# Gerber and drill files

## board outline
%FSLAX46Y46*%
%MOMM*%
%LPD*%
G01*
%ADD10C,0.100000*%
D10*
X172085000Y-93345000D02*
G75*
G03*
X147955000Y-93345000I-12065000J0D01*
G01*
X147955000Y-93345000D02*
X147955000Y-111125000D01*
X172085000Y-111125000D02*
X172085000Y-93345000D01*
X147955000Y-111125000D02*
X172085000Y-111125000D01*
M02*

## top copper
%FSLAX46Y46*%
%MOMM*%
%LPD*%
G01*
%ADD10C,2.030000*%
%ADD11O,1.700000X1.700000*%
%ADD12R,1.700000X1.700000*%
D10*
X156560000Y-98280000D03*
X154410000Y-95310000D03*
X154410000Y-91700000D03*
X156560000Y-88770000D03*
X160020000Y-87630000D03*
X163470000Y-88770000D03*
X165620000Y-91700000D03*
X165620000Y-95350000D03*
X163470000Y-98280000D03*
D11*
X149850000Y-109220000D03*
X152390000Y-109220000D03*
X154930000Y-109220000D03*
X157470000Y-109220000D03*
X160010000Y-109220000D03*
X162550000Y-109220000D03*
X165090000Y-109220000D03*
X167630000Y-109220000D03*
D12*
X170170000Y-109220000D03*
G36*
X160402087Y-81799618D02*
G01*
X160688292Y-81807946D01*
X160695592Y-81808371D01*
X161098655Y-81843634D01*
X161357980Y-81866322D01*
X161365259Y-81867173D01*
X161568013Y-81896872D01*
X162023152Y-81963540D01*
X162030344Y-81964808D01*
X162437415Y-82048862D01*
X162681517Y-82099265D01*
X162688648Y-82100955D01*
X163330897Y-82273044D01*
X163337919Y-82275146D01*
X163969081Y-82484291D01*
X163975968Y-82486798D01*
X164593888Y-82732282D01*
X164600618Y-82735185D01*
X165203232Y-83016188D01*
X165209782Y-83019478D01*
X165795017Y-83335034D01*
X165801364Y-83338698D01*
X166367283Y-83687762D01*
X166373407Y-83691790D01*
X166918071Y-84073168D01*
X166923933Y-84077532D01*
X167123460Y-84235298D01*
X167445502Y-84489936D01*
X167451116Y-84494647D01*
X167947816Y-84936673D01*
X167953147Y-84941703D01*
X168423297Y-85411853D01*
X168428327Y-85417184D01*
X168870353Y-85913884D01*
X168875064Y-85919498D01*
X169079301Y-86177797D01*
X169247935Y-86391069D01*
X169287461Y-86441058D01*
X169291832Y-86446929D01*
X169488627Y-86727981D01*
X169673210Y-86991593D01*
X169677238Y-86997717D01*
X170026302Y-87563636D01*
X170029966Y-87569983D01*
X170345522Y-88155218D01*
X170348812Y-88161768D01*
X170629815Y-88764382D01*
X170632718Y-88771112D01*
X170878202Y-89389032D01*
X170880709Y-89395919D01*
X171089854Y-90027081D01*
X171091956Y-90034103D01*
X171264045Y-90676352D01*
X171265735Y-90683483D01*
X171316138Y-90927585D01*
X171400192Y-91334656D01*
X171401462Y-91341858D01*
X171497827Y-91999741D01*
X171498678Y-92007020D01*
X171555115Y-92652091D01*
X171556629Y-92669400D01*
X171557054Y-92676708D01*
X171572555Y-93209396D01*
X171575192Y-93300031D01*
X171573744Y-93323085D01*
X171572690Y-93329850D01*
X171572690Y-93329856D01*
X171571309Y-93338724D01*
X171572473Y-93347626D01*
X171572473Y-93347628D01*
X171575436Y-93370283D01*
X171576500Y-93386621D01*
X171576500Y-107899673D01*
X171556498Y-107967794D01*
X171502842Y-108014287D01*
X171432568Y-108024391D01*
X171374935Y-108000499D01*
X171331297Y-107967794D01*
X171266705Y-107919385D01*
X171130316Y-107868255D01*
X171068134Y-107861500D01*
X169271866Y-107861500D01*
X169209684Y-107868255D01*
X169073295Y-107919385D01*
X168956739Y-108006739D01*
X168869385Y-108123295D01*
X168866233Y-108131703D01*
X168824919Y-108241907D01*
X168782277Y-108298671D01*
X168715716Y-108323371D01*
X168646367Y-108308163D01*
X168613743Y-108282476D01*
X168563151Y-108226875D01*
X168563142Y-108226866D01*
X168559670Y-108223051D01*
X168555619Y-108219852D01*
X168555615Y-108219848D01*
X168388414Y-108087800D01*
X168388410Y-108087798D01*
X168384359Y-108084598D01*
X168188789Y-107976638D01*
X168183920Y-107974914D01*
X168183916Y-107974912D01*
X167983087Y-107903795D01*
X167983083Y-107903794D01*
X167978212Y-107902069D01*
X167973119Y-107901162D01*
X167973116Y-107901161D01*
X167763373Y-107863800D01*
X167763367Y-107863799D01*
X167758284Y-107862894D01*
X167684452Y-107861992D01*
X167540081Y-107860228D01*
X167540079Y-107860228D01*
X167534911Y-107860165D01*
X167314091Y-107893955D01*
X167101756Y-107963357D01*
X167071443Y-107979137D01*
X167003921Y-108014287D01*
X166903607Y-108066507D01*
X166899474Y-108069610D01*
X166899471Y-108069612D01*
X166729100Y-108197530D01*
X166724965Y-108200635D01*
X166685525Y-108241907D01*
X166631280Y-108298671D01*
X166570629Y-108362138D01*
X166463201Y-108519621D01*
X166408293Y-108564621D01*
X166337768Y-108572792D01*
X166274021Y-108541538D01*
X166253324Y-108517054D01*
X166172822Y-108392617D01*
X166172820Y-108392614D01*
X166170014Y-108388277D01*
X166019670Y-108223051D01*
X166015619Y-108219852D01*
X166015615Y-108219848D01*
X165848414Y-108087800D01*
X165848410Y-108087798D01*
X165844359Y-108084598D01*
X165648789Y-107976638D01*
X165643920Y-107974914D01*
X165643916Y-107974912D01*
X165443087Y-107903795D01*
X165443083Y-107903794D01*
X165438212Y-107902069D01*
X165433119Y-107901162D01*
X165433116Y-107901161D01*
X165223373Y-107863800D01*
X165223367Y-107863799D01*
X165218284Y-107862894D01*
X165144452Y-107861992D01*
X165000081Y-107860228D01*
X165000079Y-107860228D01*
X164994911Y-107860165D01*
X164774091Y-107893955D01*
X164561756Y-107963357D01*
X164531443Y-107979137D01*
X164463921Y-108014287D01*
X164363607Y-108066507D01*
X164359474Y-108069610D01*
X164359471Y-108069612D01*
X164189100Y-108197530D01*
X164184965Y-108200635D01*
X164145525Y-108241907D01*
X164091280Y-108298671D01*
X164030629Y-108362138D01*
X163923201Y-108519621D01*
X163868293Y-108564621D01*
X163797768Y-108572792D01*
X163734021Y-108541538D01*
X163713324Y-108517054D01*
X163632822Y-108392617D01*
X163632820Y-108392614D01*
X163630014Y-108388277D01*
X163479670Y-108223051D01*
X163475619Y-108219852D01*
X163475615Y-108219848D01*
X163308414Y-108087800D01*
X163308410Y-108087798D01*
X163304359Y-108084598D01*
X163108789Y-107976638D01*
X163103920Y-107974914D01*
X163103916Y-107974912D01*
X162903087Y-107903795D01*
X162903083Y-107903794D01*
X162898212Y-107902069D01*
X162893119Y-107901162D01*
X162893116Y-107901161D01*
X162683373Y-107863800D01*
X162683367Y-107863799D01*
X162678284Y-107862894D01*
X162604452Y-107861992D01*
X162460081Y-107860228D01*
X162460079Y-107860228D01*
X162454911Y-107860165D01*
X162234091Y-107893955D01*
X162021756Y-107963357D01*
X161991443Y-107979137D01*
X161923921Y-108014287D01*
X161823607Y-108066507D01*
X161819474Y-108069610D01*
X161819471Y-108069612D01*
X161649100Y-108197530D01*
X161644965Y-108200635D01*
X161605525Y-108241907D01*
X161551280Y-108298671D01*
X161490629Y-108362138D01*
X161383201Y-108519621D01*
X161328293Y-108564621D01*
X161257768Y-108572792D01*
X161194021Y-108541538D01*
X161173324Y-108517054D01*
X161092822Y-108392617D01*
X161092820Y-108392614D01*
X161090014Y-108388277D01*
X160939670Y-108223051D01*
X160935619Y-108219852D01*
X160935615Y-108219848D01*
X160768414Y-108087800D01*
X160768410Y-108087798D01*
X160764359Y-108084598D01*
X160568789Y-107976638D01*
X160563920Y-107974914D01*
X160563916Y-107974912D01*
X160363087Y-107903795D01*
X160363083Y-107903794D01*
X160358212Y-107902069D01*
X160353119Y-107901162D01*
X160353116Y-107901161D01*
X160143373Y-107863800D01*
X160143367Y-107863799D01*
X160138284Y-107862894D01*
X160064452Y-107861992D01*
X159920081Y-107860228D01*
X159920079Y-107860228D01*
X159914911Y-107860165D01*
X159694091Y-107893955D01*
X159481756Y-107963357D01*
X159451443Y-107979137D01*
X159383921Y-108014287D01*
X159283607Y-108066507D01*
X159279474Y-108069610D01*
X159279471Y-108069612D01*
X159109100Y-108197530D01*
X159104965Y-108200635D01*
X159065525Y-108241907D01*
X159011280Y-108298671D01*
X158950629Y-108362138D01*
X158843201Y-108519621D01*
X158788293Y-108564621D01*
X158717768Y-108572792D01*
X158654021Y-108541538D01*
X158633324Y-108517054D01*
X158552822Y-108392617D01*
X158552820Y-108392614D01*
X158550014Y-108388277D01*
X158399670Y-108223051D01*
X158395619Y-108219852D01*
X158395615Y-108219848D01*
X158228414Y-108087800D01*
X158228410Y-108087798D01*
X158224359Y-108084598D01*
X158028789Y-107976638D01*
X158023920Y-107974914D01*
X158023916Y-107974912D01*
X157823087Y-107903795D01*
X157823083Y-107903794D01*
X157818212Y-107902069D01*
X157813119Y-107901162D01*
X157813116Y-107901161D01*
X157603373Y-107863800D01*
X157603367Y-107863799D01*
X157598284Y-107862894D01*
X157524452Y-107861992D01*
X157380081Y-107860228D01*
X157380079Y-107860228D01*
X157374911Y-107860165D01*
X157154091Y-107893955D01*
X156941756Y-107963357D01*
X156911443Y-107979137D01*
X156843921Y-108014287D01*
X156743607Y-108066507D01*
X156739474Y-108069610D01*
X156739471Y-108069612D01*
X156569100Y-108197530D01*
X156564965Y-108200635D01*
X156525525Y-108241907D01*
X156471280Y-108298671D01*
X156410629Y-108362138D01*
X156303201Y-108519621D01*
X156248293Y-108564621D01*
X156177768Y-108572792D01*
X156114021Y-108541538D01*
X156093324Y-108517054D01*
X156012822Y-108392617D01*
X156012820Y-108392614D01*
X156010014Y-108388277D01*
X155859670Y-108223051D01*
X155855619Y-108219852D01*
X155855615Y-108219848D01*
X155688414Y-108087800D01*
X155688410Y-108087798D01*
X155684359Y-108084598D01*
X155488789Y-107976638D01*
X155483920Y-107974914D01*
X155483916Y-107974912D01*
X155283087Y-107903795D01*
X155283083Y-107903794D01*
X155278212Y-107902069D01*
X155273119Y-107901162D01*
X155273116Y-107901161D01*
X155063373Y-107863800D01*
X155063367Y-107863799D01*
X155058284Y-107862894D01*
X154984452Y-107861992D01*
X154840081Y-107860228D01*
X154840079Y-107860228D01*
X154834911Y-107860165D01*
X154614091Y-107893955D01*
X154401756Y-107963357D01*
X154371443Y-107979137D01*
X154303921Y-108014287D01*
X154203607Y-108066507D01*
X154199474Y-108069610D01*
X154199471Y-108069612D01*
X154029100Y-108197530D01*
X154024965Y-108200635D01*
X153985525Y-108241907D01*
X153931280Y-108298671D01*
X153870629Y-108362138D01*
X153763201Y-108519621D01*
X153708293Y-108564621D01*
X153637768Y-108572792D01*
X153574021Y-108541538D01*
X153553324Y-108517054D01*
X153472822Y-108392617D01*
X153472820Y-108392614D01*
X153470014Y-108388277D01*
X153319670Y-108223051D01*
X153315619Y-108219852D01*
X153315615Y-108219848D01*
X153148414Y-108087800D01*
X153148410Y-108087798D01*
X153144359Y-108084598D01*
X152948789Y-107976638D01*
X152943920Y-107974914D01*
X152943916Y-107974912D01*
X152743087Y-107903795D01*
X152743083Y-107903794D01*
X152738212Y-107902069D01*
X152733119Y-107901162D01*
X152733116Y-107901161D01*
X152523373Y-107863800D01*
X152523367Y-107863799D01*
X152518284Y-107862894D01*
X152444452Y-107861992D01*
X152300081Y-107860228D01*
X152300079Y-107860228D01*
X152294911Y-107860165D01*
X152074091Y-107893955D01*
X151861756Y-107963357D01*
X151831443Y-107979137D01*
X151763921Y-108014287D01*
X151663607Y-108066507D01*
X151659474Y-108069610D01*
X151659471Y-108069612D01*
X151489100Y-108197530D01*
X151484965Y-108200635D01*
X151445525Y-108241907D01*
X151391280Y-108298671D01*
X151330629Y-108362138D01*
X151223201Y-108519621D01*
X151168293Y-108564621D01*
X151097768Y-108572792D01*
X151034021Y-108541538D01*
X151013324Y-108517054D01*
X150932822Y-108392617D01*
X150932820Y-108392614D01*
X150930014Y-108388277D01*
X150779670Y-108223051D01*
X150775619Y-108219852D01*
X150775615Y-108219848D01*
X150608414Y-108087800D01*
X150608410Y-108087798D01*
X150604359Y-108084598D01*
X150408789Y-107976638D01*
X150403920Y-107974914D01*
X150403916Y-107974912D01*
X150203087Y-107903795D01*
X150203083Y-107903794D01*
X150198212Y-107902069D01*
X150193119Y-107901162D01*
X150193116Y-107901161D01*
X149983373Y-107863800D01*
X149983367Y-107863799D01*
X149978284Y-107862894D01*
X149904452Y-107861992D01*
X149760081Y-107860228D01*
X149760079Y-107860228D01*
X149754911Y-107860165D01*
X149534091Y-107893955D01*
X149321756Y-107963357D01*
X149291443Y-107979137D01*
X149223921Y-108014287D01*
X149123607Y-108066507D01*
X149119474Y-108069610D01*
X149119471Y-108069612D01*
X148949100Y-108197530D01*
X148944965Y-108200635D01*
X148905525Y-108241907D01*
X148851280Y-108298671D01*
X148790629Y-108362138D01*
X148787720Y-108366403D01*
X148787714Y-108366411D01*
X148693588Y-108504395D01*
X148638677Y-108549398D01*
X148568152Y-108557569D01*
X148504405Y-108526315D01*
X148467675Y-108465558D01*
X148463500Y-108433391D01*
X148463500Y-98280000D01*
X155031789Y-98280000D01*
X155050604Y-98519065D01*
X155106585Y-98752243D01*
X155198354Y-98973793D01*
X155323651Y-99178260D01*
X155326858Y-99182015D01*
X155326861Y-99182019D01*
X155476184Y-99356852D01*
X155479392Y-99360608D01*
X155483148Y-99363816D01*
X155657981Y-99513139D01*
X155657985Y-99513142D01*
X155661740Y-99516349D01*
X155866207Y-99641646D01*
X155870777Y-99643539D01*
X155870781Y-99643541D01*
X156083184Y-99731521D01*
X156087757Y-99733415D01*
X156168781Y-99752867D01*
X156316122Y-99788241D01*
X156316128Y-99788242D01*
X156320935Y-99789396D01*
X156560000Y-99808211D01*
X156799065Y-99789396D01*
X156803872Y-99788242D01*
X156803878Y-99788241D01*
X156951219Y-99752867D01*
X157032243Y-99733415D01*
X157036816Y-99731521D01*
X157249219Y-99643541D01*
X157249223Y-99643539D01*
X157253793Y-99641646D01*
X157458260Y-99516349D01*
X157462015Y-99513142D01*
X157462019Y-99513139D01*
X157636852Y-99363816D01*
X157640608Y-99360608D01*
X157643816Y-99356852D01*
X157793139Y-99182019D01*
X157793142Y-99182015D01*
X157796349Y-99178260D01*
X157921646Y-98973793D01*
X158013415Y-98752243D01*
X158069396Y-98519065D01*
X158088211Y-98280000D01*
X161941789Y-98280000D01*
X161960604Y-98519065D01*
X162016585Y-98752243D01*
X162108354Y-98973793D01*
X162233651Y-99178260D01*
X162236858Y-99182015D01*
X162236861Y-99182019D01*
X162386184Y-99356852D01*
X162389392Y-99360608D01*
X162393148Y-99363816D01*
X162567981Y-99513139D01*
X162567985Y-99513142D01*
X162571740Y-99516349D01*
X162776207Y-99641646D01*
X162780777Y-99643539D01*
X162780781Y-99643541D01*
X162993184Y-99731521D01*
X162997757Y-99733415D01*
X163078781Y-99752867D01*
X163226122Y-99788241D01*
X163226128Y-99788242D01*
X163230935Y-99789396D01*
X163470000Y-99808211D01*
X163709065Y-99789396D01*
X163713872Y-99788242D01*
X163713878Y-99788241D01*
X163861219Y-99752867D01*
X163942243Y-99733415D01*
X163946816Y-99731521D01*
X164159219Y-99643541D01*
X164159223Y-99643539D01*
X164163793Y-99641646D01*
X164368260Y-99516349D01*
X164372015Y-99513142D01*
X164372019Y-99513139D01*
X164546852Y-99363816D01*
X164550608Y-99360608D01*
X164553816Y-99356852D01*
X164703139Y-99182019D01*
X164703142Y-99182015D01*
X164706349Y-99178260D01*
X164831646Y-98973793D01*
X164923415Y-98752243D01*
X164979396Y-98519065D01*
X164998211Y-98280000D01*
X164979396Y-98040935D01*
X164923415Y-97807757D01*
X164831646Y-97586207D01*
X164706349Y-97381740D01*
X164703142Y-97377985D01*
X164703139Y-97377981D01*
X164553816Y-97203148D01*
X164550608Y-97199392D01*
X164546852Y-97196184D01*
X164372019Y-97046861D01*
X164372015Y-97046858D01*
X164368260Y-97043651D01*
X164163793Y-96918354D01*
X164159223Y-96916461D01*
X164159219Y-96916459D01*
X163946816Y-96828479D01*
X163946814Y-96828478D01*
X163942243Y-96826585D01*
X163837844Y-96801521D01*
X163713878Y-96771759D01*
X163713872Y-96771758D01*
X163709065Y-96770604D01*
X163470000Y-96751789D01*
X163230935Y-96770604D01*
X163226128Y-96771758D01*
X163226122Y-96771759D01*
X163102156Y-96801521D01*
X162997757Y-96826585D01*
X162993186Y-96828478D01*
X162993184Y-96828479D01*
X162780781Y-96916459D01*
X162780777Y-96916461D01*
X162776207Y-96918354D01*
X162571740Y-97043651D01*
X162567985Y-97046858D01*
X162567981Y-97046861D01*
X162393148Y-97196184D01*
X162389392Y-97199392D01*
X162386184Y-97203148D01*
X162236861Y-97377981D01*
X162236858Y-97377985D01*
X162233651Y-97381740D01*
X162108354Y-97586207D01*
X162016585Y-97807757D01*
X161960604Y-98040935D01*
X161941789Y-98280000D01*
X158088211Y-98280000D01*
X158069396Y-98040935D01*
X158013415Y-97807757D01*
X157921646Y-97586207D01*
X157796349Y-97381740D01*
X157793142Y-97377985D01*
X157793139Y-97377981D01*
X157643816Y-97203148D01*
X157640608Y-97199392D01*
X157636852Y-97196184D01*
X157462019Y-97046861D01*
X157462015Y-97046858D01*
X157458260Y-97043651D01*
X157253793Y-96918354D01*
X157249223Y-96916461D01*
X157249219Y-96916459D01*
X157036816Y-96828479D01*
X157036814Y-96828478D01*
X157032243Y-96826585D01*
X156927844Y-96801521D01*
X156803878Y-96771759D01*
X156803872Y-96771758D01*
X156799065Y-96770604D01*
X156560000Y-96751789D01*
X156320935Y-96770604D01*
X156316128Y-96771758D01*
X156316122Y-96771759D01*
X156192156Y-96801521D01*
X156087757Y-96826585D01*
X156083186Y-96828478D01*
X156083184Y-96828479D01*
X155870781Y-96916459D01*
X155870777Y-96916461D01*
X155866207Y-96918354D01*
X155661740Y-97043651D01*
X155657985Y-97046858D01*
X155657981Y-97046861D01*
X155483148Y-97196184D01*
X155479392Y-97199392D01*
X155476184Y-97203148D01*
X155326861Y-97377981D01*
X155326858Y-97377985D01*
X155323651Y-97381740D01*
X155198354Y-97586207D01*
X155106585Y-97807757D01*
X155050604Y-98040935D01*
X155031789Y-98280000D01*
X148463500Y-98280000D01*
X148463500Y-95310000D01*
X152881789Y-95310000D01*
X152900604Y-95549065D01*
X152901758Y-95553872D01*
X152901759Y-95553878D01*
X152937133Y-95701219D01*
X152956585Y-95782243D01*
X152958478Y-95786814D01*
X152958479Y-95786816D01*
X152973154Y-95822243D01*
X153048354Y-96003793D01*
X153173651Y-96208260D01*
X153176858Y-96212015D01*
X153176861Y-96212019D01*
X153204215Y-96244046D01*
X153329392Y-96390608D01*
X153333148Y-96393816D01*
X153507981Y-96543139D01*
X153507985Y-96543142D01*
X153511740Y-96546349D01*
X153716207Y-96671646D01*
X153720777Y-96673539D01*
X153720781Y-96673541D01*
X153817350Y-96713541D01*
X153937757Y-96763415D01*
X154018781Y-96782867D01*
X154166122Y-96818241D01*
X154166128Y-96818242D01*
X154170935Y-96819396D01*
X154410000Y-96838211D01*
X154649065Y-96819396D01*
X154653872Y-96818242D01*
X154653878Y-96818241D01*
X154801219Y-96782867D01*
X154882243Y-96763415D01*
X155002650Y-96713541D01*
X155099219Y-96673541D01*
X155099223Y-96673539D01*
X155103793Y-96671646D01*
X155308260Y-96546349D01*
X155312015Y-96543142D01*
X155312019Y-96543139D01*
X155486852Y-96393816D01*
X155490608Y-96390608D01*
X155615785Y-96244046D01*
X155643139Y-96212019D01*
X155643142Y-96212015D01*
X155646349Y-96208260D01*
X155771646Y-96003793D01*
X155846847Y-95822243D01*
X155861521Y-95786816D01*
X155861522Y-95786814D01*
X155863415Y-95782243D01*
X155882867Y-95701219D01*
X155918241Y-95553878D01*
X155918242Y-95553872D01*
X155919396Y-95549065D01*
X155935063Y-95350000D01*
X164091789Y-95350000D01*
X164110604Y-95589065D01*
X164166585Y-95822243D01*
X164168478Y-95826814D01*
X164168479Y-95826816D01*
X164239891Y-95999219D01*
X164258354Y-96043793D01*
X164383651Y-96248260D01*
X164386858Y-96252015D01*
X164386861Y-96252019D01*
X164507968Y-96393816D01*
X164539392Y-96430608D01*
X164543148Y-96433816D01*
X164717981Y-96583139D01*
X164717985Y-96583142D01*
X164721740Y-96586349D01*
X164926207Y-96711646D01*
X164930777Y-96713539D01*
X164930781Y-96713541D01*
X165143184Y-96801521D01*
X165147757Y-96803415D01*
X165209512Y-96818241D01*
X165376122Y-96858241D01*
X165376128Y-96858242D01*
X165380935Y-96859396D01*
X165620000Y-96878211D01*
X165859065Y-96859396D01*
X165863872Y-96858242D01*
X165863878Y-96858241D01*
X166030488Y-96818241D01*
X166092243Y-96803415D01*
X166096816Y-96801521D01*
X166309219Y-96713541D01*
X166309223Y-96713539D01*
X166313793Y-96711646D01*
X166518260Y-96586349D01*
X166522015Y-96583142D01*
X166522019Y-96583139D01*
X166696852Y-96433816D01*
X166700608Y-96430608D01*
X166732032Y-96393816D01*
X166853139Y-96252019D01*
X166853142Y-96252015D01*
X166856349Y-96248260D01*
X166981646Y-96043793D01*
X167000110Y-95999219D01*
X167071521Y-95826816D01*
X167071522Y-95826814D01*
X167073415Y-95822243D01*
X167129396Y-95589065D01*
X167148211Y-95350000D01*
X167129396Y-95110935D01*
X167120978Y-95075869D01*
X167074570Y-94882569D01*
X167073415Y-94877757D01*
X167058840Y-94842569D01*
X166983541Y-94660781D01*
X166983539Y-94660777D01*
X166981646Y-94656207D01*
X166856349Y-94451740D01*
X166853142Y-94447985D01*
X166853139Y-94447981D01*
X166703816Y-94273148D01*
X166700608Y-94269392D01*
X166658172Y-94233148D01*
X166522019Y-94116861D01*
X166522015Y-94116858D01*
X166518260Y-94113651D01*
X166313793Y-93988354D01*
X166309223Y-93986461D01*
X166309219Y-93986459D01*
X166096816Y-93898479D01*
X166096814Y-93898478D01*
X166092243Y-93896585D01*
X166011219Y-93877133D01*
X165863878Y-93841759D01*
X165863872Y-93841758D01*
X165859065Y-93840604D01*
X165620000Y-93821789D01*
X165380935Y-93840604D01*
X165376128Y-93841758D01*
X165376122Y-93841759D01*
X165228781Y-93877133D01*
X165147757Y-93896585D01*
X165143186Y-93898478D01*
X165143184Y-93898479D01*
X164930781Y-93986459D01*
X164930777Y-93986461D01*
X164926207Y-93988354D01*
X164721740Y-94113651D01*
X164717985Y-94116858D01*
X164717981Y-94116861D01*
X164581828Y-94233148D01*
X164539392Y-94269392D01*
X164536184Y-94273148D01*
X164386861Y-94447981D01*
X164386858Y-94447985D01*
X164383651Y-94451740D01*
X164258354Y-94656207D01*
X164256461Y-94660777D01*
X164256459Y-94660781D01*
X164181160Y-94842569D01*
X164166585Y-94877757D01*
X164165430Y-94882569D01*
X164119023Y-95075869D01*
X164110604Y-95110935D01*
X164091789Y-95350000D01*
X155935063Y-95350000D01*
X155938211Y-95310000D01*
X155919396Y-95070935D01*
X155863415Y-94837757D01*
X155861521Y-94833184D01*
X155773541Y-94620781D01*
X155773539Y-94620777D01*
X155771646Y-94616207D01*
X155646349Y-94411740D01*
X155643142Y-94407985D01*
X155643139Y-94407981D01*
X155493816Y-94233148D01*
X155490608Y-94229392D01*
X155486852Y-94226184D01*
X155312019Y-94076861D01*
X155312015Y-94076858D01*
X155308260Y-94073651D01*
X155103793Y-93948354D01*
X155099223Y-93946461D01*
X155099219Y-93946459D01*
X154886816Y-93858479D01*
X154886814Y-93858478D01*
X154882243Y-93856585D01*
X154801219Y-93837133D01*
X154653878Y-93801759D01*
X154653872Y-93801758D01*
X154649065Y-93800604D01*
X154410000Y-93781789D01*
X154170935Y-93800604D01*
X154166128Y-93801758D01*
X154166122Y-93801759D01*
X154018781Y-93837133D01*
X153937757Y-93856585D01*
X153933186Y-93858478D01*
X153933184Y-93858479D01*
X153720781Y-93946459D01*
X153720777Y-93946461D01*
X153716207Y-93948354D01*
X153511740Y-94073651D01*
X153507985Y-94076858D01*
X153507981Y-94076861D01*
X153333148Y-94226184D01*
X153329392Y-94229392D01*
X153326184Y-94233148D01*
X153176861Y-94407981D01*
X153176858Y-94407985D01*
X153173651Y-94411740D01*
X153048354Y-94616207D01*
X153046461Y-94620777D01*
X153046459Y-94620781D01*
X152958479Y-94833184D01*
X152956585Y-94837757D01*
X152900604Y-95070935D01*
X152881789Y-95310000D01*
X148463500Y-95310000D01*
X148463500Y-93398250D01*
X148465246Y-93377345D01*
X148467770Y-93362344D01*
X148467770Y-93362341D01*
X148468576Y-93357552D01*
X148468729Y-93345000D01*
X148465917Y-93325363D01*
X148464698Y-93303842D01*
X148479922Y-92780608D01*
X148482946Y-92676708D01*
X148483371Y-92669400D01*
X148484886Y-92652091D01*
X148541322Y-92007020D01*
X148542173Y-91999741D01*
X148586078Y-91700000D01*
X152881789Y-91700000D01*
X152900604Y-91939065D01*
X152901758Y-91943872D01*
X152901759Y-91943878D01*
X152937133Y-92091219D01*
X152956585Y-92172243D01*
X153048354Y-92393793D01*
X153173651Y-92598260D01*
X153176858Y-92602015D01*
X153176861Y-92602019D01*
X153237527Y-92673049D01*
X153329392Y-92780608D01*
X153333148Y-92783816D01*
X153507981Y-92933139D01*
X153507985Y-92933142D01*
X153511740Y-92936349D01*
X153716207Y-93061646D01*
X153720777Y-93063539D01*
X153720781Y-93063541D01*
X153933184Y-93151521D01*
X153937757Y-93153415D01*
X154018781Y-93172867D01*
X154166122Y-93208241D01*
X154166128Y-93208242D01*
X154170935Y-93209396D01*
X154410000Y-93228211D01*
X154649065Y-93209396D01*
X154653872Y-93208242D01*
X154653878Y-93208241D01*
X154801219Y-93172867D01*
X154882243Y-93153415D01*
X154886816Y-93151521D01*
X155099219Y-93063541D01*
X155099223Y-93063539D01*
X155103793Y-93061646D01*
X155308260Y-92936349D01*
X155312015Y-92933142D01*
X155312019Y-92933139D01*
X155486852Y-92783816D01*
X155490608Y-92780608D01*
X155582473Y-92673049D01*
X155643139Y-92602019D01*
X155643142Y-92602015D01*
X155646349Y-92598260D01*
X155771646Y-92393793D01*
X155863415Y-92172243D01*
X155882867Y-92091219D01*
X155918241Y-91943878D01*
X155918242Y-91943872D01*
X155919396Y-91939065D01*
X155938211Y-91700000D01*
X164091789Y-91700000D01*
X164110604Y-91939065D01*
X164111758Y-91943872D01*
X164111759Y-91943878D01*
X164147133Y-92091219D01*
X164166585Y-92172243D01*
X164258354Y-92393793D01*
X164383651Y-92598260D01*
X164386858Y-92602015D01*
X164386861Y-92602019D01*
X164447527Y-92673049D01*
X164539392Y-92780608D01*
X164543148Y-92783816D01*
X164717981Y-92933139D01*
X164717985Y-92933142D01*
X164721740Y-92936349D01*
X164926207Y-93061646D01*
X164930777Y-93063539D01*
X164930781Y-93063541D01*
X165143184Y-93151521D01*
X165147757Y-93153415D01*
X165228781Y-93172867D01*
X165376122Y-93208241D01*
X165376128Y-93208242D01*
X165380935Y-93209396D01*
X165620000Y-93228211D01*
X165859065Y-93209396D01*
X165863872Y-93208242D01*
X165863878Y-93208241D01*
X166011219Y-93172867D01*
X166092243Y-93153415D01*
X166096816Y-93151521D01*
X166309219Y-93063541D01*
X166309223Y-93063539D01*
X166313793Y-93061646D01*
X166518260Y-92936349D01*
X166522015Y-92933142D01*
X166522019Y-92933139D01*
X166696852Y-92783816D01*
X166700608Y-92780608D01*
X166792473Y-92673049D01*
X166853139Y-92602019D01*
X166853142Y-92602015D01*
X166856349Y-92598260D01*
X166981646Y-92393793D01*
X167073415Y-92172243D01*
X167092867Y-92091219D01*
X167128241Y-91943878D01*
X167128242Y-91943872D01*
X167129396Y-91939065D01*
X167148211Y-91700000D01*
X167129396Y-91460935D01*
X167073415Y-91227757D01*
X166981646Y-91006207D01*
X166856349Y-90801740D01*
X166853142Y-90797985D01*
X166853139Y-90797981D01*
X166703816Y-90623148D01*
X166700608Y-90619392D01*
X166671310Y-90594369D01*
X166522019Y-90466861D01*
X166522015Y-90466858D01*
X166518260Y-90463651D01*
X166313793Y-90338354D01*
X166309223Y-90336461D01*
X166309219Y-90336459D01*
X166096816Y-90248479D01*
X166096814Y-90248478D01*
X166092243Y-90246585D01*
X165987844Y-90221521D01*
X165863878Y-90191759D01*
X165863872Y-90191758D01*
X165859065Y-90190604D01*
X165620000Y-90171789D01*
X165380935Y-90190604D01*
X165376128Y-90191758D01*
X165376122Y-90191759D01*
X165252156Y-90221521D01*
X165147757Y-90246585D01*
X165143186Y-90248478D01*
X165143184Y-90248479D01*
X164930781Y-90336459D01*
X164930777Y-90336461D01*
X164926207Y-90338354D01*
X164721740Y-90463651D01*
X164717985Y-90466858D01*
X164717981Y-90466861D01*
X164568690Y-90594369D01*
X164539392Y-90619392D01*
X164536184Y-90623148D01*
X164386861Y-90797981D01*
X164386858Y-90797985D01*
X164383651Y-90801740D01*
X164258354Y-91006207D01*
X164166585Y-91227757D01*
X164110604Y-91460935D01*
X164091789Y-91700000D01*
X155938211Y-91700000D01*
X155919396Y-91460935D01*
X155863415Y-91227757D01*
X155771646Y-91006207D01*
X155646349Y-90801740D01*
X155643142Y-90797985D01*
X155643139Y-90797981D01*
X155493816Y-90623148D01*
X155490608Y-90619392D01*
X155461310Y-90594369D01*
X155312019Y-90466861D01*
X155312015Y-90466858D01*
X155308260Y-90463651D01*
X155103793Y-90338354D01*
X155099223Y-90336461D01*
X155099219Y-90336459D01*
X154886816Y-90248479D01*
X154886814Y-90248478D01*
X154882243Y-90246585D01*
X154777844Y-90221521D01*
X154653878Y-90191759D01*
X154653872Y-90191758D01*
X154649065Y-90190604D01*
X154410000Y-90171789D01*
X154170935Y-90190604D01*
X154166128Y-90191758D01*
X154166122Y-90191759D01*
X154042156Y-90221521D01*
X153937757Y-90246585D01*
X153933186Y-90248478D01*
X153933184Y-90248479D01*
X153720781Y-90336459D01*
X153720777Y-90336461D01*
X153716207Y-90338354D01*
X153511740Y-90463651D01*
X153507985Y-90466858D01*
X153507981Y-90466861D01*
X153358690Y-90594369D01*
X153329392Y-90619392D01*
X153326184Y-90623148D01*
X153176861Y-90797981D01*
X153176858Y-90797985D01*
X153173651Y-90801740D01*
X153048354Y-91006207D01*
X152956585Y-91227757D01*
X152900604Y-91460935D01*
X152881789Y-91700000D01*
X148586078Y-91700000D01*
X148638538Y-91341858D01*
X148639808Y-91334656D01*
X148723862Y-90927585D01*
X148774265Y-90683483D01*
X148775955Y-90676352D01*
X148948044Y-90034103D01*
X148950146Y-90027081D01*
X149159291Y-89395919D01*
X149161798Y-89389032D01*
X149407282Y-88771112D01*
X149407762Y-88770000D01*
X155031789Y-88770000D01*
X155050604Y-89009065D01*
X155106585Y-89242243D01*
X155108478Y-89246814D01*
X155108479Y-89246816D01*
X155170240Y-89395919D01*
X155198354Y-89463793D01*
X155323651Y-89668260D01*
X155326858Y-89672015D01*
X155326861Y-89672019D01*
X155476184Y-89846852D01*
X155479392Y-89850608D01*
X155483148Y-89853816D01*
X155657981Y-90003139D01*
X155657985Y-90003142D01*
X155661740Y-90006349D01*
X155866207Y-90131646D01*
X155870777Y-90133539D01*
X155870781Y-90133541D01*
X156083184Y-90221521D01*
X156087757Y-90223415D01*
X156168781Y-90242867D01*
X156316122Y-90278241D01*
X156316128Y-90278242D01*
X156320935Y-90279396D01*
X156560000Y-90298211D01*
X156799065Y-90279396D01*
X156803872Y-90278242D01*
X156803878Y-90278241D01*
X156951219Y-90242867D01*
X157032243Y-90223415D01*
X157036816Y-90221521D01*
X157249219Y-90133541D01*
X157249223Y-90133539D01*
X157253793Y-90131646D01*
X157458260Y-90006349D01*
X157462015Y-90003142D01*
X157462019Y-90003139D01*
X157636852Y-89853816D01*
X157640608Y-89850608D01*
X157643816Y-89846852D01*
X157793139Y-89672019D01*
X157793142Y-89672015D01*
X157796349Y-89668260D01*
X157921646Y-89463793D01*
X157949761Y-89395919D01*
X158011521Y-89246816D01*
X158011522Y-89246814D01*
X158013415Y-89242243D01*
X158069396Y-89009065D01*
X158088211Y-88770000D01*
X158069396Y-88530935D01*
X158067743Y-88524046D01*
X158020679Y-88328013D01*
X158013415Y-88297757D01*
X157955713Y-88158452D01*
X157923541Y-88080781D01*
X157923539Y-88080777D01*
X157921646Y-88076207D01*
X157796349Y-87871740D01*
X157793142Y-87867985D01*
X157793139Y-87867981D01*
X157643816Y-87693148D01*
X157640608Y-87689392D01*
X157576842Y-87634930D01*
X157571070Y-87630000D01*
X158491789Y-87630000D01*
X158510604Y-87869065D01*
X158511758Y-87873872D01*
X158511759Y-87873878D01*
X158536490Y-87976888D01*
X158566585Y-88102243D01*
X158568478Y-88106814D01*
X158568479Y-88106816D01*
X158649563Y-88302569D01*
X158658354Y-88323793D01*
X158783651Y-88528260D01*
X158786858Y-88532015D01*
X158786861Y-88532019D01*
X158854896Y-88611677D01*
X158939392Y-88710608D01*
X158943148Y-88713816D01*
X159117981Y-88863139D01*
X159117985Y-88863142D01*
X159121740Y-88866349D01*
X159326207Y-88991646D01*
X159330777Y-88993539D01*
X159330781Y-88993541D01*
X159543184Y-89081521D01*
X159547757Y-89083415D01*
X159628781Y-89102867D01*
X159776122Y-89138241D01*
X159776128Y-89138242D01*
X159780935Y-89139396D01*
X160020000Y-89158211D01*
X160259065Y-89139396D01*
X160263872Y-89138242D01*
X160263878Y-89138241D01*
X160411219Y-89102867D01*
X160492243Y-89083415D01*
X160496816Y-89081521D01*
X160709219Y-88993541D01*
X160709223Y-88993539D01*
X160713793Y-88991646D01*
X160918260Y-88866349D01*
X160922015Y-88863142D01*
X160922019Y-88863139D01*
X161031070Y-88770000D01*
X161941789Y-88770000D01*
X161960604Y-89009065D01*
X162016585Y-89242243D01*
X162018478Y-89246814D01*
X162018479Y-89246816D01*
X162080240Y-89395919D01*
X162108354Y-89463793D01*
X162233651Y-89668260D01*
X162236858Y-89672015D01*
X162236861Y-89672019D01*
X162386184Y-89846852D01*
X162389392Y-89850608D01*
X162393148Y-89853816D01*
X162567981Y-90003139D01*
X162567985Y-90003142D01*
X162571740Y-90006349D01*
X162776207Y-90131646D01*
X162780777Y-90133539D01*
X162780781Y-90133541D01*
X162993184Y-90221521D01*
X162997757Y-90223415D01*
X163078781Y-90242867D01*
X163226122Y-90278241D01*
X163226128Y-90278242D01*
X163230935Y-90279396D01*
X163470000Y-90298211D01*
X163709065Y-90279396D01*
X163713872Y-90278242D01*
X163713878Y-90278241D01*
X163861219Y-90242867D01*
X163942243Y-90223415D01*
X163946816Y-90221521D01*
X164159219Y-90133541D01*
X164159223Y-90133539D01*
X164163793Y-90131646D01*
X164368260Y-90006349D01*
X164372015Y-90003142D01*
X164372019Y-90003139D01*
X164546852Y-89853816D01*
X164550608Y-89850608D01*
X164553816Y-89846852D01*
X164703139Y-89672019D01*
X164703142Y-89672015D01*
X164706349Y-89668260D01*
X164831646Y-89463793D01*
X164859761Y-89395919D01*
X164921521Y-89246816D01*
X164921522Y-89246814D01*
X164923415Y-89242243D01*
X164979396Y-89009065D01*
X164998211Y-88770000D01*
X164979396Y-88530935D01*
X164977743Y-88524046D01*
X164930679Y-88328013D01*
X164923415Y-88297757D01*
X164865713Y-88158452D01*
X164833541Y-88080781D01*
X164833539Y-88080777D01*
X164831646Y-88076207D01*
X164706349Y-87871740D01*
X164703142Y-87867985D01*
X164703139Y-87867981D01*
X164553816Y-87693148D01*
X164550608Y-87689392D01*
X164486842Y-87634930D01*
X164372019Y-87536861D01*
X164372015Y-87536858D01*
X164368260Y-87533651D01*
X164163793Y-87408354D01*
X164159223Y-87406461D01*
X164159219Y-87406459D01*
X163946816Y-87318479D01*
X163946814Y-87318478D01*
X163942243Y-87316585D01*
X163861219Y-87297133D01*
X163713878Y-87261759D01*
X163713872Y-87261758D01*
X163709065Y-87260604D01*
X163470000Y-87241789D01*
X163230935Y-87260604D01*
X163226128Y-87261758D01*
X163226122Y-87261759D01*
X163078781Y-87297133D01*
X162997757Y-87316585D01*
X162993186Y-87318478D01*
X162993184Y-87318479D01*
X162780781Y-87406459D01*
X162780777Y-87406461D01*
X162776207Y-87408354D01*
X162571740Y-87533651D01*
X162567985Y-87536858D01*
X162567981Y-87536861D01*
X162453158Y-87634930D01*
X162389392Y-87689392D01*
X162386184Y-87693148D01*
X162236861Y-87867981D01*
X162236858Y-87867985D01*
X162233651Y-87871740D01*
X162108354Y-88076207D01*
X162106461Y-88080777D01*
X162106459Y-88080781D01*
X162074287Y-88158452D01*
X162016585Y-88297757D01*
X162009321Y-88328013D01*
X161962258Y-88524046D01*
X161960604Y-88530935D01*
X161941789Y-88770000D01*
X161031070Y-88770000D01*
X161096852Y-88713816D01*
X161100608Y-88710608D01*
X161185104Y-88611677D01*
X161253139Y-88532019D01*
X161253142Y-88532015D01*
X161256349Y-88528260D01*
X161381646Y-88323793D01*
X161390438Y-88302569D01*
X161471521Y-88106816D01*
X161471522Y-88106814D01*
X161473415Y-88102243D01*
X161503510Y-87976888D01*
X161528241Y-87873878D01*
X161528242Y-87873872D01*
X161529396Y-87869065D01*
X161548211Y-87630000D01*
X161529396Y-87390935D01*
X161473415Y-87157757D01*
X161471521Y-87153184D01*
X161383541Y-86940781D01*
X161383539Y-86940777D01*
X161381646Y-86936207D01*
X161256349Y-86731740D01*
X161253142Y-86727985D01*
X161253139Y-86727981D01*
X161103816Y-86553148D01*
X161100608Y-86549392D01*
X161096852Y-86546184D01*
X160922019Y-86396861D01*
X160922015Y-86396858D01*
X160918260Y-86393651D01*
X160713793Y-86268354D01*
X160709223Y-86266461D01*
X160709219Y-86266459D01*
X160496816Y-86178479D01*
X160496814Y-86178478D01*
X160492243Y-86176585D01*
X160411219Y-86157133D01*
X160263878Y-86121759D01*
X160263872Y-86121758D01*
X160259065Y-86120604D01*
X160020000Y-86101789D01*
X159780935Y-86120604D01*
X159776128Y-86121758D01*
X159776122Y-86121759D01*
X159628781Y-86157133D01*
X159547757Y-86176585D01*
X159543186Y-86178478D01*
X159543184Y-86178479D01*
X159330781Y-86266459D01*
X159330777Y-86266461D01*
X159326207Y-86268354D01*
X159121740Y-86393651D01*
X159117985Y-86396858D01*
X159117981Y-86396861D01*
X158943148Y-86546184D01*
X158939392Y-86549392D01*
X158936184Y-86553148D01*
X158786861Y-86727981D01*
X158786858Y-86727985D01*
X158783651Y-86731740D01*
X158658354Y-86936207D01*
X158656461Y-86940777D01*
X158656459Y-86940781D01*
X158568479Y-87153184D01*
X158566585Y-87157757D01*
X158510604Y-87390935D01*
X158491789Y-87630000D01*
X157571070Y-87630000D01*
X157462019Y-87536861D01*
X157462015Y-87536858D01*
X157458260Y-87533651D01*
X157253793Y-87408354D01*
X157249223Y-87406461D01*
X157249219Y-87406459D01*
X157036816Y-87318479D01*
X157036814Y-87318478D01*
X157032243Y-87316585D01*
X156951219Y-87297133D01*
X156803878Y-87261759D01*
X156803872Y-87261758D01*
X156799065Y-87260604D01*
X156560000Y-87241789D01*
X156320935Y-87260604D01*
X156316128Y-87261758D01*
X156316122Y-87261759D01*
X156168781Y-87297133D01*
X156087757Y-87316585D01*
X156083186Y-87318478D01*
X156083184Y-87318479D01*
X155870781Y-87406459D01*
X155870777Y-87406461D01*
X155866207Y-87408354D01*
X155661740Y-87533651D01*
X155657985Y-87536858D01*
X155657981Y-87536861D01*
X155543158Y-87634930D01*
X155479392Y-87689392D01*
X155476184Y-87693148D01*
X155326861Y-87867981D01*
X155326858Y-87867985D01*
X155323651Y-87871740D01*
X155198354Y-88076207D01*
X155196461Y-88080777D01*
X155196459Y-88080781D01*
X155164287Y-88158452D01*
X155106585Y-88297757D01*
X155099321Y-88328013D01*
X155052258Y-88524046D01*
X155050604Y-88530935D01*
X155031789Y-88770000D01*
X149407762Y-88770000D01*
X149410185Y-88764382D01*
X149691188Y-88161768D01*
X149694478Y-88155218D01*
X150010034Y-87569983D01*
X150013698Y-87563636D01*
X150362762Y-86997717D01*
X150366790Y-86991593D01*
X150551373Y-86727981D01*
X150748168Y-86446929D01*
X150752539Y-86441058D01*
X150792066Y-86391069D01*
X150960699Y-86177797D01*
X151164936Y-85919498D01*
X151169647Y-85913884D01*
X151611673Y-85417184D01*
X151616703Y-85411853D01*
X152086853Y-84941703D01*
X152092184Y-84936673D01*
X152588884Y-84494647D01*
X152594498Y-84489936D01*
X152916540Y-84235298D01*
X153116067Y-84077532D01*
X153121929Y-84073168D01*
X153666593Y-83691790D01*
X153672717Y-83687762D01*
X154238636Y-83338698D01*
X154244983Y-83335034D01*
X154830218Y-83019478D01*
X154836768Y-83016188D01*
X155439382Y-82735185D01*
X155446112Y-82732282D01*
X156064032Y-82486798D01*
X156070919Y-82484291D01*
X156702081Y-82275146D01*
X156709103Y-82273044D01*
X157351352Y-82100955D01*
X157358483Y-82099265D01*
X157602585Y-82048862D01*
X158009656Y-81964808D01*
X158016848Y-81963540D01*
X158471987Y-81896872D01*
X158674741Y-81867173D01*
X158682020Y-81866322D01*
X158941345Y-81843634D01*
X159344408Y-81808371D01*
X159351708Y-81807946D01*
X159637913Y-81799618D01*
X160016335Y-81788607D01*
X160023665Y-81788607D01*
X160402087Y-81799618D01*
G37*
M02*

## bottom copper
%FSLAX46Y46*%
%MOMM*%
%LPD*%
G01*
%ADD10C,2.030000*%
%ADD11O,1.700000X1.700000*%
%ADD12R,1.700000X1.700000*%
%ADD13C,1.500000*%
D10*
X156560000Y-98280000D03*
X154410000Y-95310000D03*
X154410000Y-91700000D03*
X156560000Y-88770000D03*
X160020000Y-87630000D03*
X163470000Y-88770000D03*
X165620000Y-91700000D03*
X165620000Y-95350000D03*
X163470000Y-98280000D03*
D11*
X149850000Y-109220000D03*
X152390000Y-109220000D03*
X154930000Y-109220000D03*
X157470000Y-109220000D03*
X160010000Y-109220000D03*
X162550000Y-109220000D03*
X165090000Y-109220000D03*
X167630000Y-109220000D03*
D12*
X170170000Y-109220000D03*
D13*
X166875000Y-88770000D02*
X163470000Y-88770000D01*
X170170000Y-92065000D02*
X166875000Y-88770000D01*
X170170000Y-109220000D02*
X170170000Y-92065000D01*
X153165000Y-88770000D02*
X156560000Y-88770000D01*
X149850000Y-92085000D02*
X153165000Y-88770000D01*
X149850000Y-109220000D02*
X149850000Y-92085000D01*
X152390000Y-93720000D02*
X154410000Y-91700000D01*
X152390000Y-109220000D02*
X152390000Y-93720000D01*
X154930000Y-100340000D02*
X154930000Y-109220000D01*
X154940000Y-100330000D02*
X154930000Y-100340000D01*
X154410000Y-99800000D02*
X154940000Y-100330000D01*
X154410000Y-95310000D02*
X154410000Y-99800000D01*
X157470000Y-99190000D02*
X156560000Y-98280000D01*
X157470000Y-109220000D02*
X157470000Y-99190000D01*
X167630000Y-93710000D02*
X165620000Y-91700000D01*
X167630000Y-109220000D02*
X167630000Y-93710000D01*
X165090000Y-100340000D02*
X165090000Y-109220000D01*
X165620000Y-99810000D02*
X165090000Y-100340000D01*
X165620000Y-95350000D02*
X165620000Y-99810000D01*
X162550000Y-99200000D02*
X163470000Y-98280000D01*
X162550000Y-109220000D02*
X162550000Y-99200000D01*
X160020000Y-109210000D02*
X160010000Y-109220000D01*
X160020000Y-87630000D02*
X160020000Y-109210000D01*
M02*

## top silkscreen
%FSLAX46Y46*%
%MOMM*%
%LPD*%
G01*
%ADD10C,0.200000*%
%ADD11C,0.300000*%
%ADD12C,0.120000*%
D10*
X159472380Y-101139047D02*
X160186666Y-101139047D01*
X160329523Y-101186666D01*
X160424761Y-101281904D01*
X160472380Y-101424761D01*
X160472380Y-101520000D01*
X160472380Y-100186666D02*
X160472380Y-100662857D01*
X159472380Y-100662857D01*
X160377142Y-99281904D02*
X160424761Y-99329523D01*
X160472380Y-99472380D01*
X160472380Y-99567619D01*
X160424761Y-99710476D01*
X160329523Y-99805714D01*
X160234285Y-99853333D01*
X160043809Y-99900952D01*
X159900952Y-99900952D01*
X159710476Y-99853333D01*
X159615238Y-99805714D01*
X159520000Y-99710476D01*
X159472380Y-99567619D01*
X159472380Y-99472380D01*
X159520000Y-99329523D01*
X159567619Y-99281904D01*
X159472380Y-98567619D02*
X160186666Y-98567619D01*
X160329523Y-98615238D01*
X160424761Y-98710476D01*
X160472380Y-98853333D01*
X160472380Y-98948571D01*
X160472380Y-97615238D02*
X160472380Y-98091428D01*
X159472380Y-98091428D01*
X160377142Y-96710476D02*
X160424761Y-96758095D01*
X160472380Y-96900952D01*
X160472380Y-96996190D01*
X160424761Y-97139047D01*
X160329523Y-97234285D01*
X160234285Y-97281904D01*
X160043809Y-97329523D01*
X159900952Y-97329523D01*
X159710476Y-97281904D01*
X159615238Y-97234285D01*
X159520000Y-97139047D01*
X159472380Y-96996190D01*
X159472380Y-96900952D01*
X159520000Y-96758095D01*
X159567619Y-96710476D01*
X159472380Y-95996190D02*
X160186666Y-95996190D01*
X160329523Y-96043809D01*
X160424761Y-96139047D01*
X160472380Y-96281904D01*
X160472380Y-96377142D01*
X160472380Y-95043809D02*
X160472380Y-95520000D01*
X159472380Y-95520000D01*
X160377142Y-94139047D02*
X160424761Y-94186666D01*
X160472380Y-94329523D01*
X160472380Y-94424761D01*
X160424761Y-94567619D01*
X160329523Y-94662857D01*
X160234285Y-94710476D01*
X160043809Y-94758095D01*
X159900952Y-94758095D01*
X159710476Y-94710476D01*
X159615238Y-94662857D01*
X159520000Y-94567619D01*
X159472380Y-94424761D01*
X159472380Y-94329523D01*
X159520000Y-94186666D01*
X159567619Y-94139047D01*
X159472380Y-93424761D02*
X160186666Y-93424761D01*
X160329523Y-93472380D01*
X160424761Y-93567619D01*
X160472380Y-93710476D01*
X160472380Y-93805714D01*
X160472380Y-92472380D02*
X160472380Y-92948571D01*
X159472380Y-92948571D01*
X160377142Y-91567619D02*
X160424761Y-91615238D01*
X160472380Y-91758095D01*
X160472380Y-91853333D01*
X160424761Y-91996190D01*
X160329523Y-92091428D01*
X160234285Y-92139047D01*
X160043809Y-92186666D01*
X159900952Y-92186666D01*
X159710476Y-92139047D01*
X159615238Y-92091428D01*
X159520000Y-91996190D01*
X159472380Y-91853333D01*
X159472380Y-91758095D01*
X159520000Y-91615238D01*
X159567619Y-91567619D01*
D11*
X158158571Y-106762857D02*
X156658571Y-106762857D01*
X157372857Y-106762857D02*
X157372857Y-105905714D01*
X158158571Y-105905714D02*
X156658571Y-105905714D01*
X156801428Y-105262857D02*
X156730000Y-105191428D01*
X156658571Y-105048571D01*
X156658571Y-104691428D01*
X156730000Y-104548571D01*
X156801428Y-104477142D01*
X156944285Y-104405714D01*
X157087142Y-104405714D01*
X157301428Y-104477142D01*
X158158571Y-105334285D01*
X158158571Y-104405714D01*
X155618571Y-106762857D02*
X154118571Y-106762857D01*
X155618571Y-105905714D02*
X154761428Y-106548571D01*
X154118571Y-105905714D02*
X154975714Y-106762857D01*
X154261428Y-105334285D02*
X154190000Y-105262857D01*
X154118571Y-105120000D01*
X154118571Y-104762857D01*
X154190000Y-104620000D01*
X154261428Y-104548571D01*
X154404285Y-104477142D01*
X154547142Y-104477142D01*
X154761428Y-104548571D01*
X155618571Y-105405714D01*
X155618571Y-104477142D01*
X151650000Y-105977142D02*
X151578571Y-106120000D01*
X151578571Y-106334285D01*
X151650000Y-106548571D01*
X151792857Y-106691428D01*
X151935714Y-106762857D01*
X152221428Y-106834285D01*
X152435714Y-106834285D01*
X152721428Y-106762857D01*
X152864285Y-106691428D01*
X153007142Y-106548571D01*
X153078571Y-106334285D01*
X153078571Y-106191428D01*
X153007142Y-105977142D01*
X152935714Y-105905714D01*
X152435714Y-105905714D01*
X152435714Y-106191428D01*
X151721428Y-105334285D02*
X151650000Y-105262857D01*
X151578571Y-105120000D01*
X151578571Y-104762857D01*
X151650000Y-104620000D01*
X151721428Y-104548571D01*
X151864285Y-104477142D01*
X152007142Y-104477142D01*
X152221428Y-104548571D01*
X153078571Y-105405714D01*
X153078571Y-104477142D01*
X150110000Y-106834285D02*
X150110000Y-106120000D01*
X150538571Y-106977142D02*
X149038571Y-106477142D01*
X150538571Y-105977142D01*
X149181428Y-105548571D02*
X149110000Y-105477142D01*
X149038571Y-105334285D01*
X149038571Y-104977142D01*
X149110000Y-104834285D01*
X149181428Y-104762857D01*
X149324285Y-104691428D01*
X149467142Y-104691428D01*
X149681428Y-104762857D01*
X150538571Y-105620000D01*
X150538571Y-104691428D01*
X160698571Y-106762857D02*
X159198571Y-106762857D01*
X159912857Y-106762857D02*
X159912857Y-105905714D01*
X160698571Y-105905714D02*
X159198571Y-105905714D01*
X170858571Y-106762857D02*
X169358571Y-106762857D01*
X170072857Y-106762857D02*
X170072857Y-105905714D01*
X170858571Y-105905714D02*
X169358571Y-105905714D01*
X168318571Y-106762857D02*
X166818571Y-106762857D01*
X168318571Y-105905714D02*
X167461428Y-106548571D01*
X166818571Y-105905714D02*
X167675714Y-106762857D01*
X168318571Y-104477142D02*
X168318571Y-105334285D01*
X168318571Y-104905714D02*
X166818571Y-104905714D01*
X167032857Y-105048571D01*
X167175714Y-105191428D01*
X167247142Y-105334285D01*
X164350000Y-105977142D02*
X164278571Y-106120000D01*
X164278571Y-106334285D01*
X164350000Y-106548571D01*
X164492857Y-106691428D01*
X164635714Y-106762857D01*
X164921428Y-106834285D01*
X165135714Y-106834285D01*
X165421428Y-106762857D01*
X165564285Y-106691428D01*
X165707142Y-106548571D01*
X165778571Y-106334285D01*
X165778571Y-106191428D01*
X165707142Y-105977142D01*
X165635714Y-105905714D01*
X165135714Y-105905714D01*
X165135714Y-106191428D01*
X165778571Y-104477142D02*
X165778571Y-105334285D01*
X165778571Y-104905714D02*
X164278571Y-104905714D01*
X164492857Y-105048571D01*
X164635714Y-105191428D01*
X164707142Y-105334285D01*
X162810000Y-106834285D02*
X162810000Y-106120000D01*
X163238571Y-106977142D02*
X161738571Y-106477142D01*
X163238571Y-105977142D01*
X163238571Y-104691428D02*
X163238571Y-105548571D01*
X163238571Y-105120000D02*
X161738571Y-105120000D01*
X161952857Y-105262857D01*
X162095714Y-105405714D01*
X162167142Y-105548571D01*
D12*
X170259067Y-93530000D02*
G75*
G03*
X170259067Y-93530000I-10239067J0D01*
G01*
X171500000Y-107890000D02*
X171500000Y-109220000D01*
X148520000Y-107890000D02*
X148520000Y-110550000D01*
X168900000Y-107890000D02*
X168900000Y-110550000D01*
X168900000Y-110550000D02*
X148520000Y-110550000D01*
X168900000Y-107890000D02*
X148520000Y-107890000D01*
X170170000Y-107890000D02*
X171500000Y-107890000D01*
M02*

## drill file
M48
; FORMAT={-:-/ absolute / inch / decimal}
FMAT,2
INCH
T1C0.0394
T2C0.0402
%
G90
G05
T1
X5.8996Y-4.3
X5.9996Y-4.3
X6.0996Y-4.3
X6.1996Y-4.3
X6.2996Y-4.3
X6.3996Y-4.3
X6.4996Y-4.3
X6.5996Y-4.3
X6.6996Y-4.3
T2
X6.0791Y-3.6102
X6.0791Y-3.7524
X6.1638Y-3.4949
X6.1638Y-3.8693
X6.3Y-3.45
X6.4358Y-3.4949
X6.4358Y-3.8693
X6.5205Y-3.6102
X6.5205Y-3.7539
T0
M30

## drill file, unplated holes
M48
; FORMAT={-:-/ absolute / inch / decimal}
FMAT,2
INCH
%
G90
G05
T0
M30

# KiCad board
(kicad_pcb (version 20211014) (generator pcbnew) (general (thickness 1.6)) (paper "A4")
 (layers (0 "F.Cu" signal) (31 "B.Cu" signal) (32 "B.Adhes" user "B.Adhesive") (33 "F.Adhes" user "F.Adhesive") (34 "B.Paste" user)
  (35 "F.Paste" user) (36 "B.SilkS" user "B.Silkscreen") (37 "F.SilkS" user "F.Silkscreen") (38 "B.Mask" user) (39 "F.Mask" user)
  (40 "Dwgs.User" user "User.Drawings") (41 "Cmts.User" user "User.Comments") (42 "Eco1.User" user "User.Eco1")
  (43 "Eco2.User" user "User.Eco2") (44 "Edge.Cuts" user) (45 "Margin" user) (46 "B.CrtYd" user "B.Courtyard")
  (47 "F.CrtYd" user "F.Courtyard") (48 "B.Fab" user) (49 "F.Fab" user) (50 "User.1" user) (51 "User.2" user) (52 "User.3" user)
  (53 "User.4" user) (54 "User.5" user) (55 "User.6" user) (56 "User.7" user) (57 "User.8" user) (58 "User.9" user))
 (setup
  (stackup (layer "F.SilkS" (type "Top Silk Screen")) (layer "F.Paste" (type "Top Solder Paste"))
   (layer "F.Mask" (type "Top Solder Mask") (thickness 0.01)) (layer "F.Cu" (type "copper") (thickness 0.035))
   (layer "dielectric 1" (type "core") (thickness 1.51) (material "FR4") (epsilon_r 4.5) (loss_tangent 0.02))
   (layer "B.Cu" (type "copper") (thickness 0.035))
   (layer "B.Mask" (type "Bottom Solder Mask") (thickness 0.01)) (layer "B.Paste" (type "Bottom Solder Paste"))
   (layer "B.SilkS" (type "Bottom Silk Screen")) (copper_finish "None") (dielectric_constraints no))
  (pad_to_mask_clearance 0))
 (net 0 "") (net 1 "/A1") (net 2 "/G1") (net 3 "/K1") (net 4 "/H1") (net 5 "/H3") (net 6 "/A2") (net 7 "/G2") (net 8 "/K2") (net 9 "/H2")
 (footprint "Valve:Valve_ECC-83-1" (layer "F.Cu") (at 163.47 98.28)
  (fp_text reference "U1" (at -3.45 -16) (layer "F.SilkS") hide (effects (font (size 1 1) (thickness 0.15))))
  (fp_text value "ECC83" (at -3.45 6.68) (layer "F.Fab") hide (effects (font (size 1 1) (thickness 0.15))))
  (fp_circle (center -3.45 -4.75) (end 6.71 -3.48) (layer "F.SilkS") (width 0.12) (fill none))
  (pad "1" thru_hole circle (at 0 0) (size 2.03 2.03) (drill 1.02) (layers *.Cu *.Mask) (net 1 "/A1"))
  (pad "2" thru_hole circle (at 2.15 -2.93) (size 2.03 2.03) (drill 1.02) (layers *.Cu *.Mask) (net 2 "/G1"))
  (pad "3" thru_hole circle (at 2.15 -6.58) (size 2.03 2.03) (drill 1.02) (layers *.Cu *.Mask) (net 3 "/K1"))
  (pad "4" thru_hole circle (at 0 -9.51) (size 2.03 2.03) (drill 1.02) (layers *.Cu *.Mask) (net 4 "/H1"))
  (pad "5" thru_hole circle (at -3.45 -10.65) (size 2.03 2.03) (drill 1.02) (layers *.Cu *.Mask) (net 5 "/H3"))
  (pad "6" thru_hole circle (at -6.91 -9.51) (size 2.03 2.03) (drill 1.02) (layers *.Cu *.Mask) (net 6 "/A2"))
  (pad "7" thru_hole circle (at -9.06 -6.58) (size 2.03 2.03) (drill 1.02) (layers *.Cu *.Mask) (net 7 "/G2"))
  (pad "8" thru_hole circle (at -9.06 -2.97) (size 2.03 2.03) (drill 1.02) (layers *.Cu *.Mask) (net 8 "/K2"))
  (pad "9" thru_hole circle (at -6.91 0) (size 2.03 2.03) (drill 1.02) (layers *.Cu *.Mask) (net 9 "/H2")))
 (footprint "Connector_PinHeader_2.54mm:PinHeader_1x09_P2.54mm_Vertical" (layer "F.Cu") (at 170.17 109.22 -90)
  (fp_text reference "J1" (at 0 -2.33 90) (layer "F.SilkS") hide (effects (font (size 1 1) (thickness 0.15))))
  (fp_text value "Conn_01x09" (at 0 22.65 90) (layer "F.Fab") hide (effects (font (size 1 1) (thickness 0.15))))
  (fp_line (start -1.33 1.27) (end 1.33 1.27) (layer "F.SilkS") (width 0.12))
  (fp_line (start -1.33 21.65) (end 1.33 21.65) (layer "F.SilkS") (width 0.12))
  (fp_line (start -1.33 0) (end -1.33 -1.33) (layer "F.SilkS") (width 0.12))
  (fp_line (start -1.33 1.27) (end -1.33 21.65) (layer "F.SilkS") (width 0.12))
  (fp_line (start -1.33 -1.33) (end 0 -1.33) (layer "F.SilkS") (width 0.12))
  (fp_line (start 1.33 1.27) (end 1.33 21.65) (layer "F.SilkS") (width 0.12))
  (pad "1" thru_hole rect (at 0 0 270) (size 1.7 1.7) (drill 1) (layers *.Cu *.Mask) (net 4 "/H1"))
  (pad "2" thru_hole oval (at 0 2.54 270) (size 1.7 1.7) (drill 1) (layers *.Cu *.Mask) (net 3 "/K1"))
  (pad "3" thru_hole oval (at 0 5.08 270) (size 1.7 1.7) (drill 1) (layers *.Cu *.Mask) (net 2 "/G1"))
  (pad "4" thru_hole oval (at 0 7.62 270) (size 1.7 1.7) (drill 1) (layers *.Cu *.Mask) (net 1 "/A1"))
  (pad "5" thru_hole oval (at 0 10.16 270) (size 1.7 1.7) (drill 1) (layers *.Cu *.Mask) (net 5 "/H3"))
  (pad "6" thru_hole oval (at 0 12.7 270) (size 1.7 1.7) (drill 1) (layers *.Cu *.Mask) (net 9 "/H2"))
  (pad "7" thru_hole oval (at 0 15.24 270) (size 1.7 1.7) (drill 1) (layers *.Cu *.Mask) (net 8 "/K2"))
  (pad "8" thru_hole oval (at 0 17.78 270) (size 1.7 1.7) (drill 1) (layers *.Cu *.Mask) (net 7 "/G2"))
  (pad "9" thru_hole oval (at 0 20.32 270) (size 1.7 1.7) (drill 1) (layers *.Cu *.Mask) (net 6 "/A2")))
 (gr_arc (start 147.955 93.345) (mid 160.02 81.28) (end 172.085 93.345) (layer "Edge.Cuts") (width 0.1))
 (gr_line (start 147.955 93.345) (end 147.955 111.125) (layer "Edge.Cuts") (width 0.1))
 (gr_line (start 172.085 111.125) (end 172.085 93.345) (layer "Edge.Cuts") (width 0.1))
 (gr_line (start 147.955 111.125) (end 172.085 111.125) (layer "Edge.Cuts") (width 0.1))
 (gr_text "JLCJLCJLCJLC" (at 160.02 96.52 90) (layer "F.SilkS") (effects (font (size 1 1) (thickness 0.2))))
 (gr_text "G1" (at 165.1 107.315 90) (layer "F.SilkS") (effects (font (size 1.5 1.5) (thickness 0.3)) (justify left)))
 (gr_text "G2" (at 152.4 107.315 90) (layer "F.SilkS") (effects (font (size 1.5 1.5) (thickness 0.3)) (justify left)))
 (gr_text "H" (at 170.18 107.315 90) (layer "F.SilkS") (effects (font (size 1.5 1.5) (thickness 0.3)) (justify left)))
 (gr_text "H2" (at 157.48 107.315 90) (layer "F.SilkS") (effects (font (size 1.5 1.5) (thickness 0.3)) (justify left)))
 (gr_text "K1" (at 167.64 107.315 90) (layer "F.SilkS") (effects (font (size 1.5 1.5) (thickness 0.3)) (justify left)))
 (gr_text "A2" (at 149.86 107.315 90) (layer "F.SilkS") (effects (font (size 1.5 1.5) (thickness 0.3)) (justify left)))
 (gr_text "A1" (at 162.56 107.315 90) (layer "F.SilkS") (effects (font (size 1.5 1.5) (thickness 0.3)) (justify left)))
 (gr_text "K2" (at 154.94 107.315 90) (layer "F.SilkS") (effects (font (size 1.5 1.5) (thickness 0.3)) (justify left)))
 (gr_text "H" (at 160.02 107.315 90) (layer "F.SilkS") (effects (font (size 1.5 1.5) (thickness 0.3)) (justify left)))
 (segment (start 162.55 99.2) (end 163.47 98.28) (width 1.5) (layer "B.Cu") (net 1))
 (segment (start 162.55 109.22) (end 162.55 99.2) (width 1.5) (layer "B.Cu") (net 1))
 (segment (start 165.62 99.81) (end 165.09 100.34) (width 1.5) (layer "B.Cu") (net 2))
 (segment (start 165.62 95.35) (end 165.62 99.81) (width 1.5) (layer "B.Cu") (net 2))
 (segment (start 165.09 100.34) (end 165.09 109.22) (width 1.5) (layer "B.Cu") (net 2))
 (segment (start 167.63 93.71) (end 165.62 91.7) (width 1.5) (layer "B.Cu") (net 3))
 (segment (start 167.63 109.22) (end 167.63 93.71) (width 1.5) (layer "B.Cu") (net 3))
 (segment (start 170.17 109.22) (end 170.17 92.065) (width 1.5) (layer "B.Cu") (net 4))
 (segment (start 170.17 92.065) (end 166.875 88.77) (width 1.5) (layer "B.Cu") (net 4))
 (segment (start 166.875 88.77) (end 163.47 88.77) (width 1.5) (layer "B.Cu") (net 4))
 (segment (start 157.47 109.22) (end 157.47 99.19) (width 1.5) (layer "B.Cu") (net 9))
 (segment (start 157.47 99.19) (end 156.56 98.28) (width 1.5) (layer "B.Cu") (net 9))
 (segment (start 149.85 92.085) (end 153.165 88.77) (width 1.5) (layer "B.Cu") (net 6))
 (segment (start 153.165 88.77) (end 156.56 88.77) (width 1.5) (layer "B.Cu") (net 6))
 (segment (start 149.85 109.22) (end 149.85 92.085) (width 1.5) (layer "B.Cu") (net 6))
 (segment (start 152.39 93.72) (end 154.41 91.7) (width 1.5) (layer "B.Cu") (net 7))
 (segment (start 152.39 109.22) (end 152.39 93.72) (width 1.5) (layer "B.Cu") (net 7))
 (segment (start 154.41 95.31) (end 154.41 99.8) (width 1.5) (layer "B.Cu") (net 8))
 (segment (start 154.93 100.34) (end 154.93 109.22) (width 1.5) (layer "B.Cu") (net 8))
 (segment (start 154.94 100.33) (end 154.93 100.34) (width 1.5) (layer "B.Cu") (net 8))
 (segment (start 154.41 99.8) (end 154.94 100.33) (width 1.5) (layer "B.Cu") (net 8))
 (segment (start 160.02 87.63) (end 160.02 109.21) (width 1.5) (layer "B.Cu") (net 5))
 (segment (start 160.02 109.21) (end 160.01 109.22) (width 1.5) (layer "B.Cu") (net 5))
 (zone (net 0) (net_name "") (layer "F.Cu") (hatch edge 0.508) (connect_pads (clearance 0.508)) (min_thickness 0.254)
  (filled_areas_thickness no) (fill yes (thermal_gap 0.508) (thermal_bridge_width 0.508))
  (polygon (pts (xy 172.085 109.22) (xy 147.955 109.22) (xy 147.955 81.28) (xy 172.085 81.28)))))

